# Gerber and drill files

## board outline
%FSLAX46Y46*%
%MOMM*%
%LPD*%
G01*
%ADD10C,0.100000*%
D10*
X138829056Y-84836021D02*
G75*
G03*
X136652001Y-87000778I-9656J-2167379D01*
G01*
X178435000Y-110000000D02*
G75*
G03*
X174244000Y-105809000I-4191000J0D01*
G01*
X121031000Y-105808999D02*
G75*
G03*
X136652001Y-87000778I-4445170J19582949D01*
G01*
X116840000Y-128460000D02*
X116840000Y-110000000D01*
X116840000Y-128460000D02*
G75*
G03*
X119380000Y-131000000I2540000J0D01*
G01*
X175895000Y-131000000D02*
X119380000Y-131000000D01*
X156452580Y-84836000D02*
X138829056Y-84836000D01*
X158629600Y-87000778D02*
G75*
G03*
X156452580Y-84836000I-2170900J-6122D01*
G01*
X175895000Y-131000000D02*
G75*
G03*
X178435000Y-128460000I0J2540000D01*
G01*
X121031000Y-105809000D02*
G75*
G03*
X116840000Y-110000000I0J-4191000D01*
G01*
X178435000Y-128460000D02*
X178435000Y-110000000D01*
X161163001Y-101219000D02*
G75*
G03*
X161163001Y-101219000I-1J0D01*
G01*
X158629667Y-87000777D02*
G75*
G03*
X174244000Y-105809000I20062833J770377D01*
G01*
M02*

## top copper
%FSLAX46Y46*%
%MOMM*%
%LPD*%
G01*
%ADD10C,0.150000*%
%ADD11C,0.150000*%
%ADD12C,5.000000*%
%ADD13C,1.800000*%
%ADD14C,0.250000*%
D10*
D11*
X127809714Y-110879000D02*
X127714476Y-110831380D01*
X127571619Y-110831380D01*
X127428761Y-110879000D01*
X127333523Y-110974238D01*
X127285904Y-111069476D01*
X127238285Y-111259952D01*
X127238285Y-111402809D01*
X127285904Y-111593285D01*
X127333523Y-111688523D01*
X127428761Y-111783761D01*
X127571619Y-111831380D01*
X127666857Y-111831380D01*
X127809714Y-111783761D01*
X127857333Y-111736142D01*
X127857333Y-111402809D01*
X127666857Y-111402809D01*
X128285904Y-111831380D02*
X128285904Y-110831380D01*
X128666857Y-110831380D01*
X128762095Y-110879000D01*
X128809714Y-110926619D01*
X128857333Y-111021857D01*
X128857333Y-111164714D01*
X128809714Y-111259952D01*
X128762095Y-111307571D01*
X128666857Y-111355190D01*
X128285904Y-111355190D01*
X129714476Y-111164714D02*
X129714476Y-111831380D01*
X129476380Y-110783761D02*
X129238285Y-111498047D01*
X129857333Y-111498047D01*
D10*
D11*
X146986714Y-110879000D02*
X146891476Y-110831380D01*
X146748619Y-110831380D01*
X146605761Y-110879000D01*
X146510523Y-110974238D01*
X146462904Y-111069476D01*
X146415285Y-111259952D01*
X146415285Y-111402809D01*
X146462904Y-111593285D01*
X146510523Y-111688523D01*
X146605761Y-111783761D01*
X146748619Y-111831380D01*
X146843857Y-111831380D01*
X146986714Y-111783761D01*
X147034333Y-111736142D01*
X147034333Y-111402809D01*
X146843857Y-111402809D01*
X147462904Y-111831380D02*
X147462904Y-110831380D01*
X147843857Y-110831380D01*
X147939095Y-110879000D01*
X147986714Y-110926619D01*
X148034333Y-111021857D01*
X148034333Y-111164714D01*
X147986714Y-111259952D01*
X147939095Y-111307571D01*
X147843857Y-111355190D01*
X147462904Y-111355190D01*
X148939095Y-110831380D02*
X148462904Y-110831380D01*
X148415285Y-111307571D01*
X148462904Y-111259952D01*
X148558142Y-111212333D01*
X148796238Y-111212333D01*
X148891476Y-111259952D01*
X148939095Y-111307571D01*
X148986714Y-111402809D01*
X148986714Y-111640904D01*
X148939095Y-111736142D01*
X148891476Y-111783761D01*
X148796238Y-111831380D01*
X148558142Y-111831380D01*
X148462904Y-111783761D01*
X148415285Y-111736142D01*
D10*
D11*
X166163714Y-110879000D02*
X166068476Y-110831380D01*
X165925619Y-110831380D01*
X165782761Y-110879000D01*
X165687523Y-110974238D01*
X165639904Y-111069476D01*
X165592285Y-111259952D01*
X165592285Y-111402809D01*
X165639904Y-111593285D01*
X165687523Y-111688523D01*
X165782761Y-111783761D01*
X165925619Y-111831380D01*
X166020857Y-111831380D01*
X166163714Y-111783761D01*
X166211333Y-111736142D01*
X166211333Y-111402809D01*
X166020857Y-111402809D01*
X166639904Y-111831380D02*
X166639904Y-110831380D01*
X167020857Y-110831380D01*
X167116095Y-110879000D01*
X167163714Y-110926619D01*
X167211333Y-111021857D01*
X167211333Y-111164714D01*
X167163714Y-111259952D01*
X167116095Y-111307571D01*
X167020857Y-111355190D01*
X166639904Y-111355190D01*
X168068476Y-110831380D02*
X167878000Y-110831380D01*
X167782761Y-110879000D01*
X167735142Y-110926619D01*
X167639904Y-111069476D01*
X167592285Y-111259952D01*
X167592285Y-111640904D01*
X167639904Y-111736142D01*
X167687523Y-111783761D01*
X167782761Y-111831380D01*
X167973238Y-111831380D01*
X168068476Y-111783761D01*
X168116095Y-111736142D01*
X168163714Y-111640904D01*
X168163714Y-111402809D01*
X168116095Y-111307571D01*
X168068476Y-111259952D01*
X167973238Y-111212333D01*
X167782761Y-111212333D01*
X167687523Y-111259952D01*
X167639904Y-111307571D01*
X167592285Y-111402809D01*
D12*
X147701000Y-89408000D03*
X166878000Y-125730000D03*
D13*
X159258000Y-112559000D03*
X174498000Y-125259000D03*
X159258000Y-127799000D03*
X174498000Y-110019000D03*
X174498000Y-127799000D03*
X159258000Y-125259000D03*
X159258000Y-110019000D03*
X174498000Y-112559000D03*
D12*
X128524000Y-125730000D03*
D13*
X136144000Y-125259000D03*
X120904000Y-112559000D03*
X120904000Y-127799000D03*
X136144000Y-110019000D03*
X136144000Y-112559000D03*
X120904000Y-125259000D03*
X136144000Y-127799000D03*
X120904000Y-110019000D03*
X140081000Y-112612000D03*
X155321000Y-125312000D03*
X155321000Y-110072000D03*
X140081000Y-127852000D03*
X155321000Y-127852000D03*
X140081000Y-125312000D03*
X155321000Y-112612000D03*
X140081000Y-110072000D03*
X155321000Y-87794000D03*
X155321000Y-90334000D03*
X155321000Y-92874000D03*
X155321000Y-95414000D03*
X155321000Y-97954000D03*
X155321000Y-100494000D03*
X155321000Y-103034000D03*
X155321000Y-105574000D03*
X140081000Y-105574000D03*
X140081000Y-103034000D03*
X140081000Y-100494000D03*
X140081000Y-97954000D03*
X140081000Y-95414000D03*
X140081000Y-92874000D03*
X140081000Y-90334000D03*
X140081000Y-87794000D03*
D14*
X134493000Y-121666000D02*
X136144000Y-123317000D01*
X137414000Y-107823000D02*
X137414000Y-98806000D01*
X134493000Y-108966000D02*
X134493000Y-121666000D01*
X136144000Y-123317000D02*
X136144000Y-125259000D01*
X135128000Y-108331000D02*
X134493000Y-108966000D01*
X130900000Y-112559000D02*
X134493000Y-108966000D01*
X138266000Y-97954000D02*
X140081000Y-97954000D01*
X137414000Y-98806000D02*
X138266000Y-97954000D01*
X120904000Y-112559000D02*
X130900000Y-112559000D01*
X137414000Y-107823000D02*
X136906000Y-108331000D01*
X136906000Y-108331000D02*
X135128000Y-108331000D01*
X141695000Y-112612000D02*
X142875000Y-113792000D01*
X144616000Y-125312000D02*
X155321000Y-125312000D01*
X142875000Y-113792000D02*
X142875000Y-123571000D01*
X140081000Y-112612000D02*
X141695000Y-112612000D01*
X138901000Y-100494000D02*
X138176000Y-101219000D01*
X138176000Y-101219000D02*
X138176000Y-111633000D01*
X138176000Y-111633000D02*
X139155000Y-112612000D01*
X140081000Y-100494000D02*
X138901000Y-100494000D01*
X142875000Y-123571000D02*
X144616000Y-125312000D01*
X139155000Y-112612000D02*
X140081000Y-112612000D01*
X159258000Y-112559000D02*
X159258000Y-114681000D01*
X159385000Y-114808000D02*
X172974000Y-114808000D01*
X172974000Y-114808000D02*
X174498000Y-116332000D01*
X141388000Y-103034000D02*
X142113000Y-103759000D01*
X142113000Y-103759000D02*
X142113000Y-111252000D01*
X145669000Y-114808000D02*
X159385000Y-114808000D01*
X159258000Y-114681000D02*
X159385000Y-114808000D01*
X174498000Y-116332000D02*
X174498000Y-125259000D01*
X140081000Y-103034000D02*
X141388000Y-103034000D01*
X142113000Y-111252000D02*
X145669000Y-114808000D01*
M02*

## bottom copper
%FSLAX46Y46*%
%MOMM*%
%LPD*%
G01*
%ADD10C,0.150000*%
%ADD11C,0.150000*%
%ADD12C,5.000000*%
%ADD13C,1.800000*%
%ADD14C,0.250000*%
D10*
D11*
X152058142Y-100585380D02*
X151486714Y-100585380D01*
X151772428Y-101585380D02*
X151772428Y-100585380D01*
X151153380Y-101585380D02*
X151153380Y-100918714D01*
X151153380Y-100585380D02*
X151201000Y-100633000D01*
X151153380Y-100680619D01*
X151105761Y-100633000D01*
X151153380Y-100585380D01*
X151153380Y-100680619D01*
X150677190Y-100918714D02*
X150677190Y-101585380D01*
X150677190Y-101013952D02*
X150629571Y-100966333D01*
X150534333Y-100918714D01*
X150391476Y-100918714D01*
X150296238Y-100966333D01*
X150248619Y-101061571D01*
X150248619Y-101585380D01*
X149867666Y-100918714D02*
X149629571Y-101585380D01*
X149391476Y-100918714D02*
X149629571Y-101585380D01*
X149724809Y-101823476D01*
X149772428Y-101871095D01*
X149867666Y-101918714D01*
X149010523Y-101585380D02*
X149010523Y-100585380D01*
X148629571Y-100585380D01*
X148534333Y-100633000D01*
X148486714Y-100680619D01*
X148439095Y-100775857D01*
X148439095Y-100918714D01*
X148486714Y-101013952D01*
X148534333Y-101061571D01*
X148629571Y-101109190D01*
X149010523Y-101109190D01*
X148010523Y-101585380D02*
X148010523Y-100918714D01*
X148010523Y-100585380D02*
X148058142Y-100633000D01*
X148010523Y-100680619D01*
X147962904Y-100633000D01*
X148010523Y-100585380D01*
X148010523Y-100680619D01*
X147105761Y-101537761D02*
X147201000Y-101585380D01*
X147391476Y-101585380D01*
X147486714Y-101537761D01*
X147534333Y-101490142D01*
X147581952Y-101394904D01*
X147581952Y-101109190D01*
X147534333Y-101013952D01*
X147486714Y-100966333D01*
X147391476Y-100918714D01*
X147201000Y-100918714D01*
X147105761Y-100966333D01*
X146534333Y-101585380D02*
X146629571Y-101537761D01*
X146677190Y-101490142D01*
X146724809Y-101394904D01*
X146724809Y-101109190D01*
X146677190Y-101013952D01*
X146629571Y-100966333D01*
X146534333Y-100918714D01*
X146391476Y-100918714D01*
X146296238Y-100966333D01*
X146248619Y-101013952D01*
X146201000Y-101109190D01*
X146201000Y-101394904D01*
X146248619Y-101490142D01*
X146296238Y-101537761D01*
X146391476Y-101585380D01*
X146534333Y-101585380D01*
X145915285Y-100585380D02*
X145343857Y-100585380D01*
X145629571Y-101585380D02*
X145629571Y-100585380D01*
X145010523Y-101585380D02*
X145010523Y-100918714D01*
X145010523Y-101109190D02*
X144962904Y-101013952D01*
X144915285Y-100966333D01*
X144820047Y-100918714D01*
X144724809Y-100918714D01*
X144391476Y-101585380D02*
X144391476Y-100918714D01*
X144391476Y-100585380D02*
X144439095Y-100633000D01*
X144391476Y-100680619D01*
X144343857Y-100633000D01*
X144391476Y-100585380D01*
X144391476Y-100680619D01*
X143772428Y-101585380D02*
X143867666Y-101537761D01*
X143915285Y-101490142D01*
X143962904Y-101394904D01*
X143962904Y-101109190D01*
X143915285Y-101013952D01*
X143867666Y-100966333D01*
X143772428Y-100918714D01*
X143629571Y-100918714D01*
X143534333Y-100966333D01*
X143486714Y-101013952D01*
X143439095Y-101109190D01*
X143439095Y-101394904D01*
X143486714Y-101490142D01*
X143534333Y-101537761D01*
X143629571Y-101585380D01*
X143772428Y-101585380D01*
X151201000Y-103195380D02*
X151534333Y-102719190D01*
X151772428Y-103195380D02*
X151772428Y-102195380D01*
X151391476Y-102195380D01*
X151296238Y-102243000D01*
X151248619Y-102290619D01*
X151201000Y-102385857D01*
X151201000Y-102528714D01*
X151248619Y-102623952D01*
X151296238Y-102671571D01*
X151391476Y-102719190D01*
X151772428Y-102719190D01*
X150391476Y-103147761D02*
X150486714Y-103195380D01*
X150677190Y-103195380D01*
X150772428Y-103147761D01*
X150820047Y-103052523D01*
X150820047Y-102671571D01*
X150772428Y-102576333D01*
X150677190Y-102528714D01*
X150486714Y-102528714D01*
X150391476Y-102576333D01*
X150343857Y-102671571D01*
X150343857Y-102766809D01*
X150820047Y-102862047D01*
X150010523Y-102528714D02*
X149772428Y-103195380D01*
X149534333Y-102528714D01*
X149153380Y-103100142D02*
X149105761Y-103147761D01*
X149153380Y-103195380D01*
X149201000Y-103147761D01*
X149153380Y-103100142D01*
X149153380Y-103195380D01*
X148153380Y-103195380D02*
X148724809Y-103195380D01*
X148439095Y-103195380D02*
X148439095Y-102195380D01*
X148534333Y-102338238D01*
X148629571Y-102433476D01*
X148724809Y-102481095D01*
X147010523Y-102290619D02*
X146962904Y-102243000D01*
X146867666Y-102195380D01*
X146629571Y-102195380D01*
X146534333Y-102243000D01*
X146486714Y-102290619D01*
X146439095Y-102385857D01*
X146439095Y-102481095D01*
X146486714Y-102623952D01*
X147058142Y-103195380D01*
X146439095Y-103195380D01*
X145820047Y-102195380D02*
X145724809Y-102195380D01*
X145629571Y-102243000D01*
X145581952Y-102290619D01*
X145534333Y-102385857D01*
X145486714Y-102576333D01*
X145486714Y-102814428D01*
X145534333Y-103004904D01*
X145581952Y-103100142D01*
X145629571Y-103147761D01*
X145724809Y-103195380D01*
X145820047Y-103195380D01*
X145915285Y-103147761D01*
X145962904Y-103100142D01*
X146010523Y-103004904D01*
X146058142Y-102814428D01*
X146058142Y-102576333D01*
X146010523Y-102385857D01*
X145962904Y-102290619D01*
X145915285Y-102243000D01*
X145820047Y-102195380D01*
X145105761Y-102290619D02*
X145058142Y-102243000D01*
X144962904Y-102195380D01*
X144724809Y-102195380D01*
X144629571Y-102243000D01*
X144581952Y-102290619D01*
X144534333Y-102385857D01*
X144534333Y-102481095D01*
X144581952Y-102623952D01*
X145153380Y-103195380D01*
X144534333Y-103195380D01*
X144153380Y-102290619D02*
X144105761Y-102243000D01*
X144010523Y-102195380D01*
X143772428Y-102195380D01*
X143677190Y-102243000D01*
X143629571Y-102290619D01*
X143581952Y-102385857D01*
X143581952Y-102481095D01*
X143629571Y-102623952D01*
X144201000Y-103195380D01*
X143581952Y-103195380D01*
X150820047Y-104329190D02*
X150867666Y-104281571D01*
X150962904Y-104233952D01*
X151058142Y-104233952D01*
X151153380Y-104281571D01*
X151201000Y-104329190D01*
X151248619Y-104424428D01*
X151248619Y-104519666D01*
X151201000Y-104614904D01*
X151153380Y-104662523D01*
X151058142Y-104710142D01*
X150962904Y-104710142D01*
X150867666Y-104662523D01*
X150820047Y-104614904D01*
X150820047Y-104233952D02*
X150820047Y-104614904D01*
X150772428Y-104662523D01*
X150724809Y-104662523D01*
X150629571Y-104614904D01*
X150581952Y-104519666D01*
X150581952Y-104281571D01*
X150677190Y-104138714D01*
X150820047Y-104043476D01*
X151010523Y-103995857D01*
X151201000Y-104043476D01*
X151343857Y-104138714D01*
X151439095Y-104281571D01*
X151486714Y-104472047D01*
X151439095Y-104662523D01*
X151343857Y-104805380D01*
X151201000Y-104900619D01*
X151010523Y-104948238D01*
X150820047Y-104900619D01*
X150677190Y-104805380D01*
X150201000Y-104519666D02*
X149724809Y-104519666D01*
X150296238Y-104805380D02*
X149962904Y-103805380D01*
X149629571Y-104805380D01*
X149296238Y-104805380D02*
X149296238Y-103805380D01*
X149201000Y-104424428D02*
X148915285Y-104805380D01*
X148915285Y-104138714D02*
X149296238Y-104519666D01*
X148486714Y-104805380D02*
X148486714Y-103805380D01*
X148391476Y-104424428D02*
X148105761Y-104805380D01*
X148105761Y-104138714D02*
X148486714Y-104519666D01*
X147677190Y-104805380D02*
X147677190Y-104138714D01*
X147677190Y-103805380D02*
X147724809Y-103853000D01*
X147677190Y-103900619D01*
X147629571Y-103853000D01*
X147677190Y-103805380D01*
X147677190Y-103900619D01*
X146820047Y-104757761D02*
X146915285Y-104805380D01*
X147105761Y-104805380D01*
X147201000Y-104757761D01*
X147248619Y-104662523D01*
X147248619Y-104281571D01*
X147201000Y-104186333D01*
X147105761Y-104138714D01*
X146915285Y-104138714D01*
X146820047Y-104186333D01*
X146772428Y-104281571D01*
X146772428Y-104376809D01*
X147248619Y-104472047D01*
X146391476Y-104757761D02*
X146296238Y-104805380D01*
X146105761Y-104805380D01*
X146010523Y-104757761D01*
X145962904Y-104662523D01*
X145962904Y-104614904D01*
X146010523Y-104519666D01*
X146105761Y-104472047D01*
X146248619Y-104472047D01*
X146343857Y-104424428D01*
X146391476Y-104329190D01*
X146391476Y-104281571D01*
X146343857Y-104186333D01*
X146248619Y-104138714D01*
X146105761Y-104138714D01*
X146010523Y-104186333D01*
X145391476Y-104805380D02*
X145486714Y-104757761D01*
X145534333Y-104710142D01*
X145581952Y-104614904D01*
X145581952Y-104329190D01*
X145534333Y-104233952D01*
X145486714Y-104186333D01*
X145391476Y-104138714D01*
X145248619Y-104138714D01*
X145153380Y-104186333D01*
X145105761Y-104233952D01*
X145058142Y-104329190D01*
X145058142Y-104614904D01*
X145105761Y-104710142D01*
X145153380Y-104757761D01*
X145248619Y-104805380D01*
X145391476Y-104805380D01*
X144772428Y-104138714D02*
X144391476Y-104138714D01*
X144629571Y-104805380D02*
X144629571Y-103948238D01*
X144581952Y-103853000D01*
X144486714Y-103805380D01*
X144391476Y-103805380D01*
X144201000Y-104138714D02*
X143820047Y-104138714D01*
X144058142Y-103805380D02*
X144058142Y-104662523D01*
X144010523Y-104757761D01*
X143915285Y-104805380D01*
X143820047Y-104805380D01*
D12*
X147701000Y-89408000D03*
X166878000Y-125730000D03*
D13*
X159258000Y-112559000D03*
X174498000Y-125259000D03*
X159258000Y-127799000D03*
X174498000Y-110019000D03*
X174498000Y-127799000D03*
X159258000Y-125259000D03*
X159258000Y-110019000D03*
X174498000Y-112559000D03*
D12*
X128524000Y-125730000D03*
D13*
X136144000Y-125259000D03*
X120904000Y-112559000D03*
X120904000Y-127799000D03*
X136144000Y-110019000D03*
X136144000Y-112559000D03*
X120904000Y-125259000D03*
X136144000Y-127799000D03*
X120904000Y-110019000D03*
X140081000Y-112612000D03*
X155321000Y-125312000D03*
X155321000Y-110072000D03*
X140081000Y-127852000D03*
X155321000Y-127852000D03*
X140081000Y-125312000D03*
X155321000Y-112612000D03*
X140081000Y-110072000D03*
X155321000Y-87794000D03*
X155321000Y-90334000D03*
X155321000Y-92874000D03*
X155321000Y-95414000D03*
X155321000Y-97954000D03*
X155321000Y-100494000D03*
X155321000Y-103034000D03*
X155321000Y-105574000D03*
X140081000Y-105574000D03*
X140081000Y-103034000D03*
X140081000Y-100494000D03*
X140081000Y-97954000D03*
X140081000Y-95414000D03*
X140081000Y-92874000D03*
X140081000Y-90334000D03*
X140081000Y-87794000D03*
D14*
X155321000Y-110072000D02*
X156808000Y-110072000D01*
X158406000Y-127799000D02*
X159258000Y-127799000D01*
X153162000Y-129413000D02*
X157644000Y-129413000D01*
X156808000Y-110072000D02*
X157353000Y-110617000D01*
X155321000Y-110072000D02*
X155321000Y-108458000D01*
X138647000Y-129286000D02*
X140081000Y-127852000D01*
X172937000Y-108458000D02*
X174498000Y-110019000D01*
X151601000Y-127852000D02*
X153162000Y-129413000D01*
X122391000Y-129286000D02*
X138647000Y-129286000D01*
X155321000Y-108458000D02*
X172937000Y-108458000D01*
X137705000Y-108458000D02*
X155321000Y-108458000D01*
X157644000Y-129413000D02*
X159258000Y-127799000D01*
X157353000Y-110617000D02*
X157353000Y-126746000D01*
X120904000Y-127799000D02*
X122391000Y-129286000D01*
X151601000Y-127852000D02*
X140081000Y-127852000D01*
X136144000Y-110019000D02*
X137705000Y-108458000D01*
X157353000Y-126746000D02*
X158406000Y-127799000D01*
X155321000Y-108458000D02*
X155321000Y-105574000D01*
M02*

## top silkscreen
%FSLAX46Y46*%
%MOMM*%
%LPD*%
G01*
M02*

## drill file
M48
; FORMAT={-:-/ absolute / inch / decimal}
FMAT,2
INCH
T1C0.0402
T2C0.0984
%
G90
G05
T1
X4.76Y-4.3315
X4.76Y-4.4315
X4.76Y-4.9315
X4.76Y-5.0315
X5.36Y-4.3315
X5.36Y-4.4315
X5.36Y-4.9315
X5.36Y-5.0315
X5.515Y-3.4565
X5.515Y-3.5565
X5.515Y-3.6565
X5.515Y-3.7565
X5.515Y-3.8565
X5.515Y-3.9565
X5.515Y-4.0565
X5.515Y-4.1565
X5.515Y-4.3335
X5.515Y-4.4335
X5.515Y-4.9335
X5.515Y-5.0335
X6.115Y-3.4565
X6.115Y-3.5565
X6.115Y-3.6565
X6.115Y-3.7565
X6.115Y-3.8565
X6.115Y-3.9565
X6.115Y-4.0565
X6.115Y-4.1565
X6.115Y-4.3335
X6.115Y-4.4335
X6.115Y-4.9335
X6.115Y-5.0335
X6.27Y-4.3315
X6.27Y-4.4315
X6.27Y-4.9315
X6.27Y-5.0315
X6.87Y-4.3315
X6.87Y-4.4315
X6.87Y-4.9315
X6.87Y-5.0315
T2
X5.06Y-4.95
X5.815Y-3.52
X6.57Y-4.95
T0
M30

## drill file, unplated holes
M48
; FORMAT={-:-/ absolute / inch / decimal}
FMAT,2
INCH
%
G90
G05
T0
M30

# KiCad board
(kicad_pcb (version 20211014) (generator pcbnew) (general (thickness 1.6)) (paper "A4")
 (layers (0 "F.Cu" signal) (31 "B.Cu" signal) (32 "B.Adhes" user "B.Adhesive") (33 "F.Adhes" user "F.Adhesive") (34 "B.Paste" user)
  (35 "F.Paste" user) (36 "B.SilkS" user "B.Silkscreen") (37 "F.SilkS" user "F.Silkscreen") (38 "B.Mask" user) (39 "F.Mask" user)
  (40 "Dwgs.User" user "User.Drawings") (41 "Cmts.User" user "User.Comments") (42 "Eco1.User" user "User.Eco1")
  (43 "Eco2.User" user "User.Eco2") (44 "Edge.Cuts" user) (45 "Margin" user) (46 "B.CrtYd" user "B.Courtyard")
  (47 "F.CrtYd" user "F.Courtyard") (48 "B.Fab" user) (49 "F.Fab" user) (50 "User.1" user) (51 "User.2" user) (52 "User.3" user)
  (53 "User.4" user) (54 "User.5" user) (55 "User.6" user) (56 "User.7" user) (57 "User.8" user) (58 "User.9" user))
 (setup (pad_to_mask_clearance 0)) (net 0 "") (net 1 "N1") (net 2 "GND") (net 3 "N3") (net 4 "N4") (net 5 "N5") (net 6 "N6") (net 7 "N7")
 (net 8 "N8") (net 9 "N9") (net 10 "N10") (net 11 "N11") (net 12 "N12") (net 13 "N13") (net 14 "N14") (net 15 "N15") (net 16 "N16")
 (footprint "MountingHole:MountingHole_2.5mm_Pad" (layer "F.Cu") (at 147.701 89.408)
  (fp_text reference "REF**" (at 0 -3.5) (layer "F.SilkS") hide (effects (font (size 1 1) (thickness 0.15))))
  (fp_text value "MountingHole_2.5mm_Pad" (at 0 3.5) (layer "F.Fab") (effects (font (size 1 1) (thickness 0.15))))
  (pad "1" thru_hole circle (at 0 0) (size 5 5) (drill 2.5) (layers *.Cu *.Mask)))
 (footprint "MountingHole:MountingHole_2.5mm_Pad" (layer "F.Cu") (at 166.878 125.73)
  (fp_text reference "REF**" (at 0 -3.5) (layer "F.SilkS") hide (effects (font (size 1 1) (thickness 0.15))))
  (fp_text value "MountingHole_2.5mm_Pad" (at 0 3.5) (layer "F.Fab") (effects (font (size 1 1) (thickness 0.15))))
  (pad "1" thru_hole circle (at 0 0) (size 5 5) (drill 2.5) (layers *.Cu *.Mask)))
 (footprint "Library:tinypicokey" (layer "F.Cu") (at 166.878 104.939)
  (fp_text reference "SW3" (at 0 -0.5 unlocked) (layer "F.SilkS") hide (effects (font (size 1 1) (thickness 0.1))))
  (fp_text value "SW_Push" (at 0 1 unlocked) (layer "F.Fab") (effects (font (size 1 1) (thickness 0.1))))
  (pad "1" thru_hole circle (at -7.62 7.62) (size 1.8 1.8) (drill 1.02) (layers *.Cu *.Mask) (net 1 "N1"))
  (pad "1" thru_hole circle (at 7.62 20.32) (size 1.8 1.8) (drill 1.02) (layers *.Cu *.Mask) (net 1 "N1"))
  (pad "2" thru_hole circle (at -7.62 22.86) (size 1.8 1.8) (drill 1.02) (layers *.Cu *.Mask) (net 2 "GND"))
  (pad "2" thru_hole circle (at 7.62 5.08) (size 1.8 1.8) (drill 1.02) (layers *.Cu *.Mask) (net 2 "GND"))
  (pad "3" thru_hole circle (at 7.62 22.86) (size 1.8 1.8) (drill 1.02) (layers *.Cu *.Mask))
  (pad "3" thru_hole circle (at -7.62 20.32) (size 1.8 1.8) (drill 1.02) (layers *.Cu *.Mask))
  (pad "3" thru_hole circle (at -7.62 5.08) (size 1.8 1.8) (drill 1.02) (layers *.Cu *.Mask))
  (pad "3" thru_hole circle (at 7.62 7.62) (size 1.8 1.8) (drill 1.02) (layers *.Cu *.Mask)))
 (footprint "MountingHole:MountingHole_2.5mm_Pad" (layer "F.Cu") (at 128.524 125.73)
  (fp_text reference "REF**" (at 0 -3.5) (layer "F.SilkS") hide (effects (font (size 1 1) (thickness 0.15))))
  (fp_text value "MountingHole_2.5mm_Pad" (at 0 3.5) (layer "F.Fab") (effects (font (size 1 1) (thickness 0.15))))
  (pad "1" thru_hole circle (at 0 0) (size 5 5) (drill 2.5) (layers *.Cu *.Mask)))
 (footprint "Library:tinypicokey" (layer "F.Cu") (at 128.524 104.939)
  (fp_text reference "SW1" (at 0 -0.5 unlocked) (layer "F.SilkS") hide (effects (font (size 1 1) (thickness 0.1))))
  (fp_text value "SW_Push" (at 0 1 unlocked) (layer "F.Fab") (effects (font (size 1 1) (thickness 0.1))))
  (pad "1" thru_hole circle (at 7.62 20.32) (size 1.8 1.8) (drill 1.02) (layers *.Cu *.Mask) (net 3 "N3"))
  (pad "1" thru_hole circle (at -7.62 7.62) (size 1.8 1.8) (drill 1.02) (layers *.Cu *.Mask) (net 3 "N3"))
  (pad "2" thru_hole circle (at -7.62 22.86) (size 1.8 1.8) (drill 1.02) (layers *.Cu *.Mask) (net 2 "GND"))
  (pad "2" thru_hole circle (at 7.62 5.08) (size 1.8 1.8) (drill 1.02) (layers *.Cu *.Mask) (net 2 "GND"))
  (pad "3" thru_hole circle (at 7.62 7.62) (size 1.8 1.8) (drill 1.02) (layers *.Cu *.Mask))
  (pad "3" thru_hole circle (at -7.62 20.32) (size 1.8 1.8) (drill 1.02) (layers *.Cu *.Mask))
  (pad "3" thru_hole circle (at 7.62 22.86) (size 1.8 1.8) (drill 1.02) (layers *.Cu *.Mask))
  (pad "3" thru_hole circle (at -7.62 5.08) (size 1.8 1.8) (drill 1.02) (layers *.Cu *.Mask)))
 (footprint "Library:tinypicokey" (layer "F.Cu") (at 147.701 132.932 180)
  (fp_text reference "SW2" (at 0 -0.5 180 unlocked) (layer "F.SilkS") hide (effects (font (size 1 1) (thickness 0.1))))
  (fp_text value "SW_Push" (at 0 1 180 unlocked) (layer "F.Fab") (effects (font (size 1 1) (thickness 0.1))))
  (pad "1" thru_hole circle (at 7.62 20.32 180) (size 1.8 1.8) (drill 1.02) (layers *.Cu *.Mask) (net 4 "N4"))
  (pad "1" thru_hole circle (at -7.62 7.62 180) (size 1.8 1.8) (drill 1.02) (layers *.Cu *.Mask) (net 4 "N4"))
  (pad "2" thru_hole circle (at -7.62 22.86 180) (size 1.8 1.8) (drill 1.02) (layers *.Cu *.Mask) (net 2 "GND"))
  (pad "2" thru_hole circle (at 7.62 5.08 180) (size 1.8 1.8) (drill 1.02) (layers *.Cu *.Mask) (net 2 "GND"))
  (pad "3" thru_hole circle (at -7.62 5.08 180) (size 1.8 1.8) (drill 1.02) (layers *.Cu *.Mask))
  (pad "3" thru_hole circle (at 7.62 7.62 180) (size 1.8 1.8) (drill 1.02) (layers *.Cu *.Mask))
  (pad "3" thru_hole circle (at -7.62 20.32 180) (size 1.8 1.8) (drill 1.02) (layers *.Cu *.Mask))
  (pad "3" thru_hole circle (at 7.62 22.86 180) (size 1.8 1.8) (drill 1.02) (layers *.Cu *.Mask)))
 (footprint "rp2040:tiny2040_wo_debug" (layer "B.Cu") (at 147.701 82.714 180)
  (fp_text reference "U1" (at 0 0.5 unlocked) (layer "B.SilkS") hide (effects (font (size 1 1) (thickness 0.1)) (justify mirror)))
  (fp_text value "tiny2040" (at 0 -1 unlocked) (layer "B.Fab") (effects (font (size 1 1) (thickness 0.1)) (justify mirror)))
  (pad "1" thru_hole circle locked (at -7.62 -5.08 180) (size 1.8 1.8) (drill 1.02) (layers *.Cu *.Mask) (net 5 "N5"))
  (pad "2" thru_hole circle locked (at -7.62 -7.62 180) (size 1.8 1.8) (drill 1.02) (layers *.Cu *.Mask) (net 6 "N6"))
  (pad "3" thru_hole circle locked (at -7.62 -10.16 180) (size 1.8 1.8) (drill 1.02) (layers *.Cu *.Mask) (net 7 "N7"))
  (pad "4" thru_hole circle locked (at -7.62 -12.7 180) (size 1.8 1.8) (drill 1.02) (layers *.Cu *.Mask) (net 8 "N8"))
  (pad "5" thru_hole circle locked (at -7.62 -15.24 180) (size 1.8 1.8) (drill 1.02) (layers *.Cu *.Mask) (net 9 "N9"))
  (pad "6" thru_hole circle locked (at -7.62 -17.78 180) (size 1.8 1.8) (drill 1.02) (layers *.Cu *.Mask) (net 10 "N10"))
  (pad "7" thru_hole circle locked (at -7.62 -20.32 180) (size 1.8 1.8) (drill 1.02) (layers *.Cu *.Mask) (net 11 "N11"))
  (pad "8" thru_hole circle locked (at -7.62 -22.86 180) (size 1.8 1.8) (drill 1.02) (layers *.Cu *.Mask) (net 2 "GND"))
  (pad "9" thru_hole circle locked (at 7.62 -22.86 180) (size 1.8 1.8) (drill 1.02) (layers *.Cu *.Mask) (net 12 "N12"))
  (pad "10" thru_hole circle locked (at 7.62 -20.32 180) (size 1.8 1.8) (drill 1.02) (layers *.Cu *.Mask) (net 1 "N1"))
  (pad "11" thru_hole circle locked (at 7.62 -17.78 180) (size 1.8 1.8) (drill 1.02) (layers *.Cu *.Mask) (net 4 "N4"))
  (pad "12" thru_hole circle locked (at 7.62 -15.24 180) (size 1.8 1.8) (drill 1.02) (layers *.Cu *.Mask) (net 3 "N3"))
  (pad "13" thru_hole circle locked (at 7.62 -12.7 180) (size 1.8 1.8) (drill 1.02) (layers *.Cu *.Mask) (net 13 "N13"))
  (pad "14" thru_hole circle locked (at 7.62 -10.16 180) (size 1.8 1.8) (drill 1.02) (layers *.Cu *.Mask) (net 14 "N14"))
  (pad "15" thru_hole circle locked (at 7.62 -7.62 180) (size 1.8 1.8) (drill 1.02) (layers *.Cu *.Mask) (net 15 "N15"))
  (pad "16" thru_hole circle locked (at 7.62 -5.08 180) (size 1.8 1.8) (drill 1.02) (layers *.Cu *.Mask) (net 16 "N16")))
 (gr_arc (start 136.652001 87.000778) (mid 137.291161 85.466473) (end 138.829056 84.836) (layer "Edge.Cuts") (width 0.1))
 (gr_arc (start 174.244 105.809) (mid 177.207485 107.036515) (end 178.435 110) (layer "Edge.Cuts") (width 0.1))
 (gr_arc (start 136.652001 87.000778) (mid 132.033766 99.056197) (end 121.031 105.809) (layer "Edge.Cuts") (width 0.1))
 (gr_line (start 116.84 128.46) (end 116.84 110) (layer "Edge.Cuts") (width 0.1))
 (gr_arc (start 119.38 131) (mid 117.583949 130.256051) (end 116.84 128.46) (layer "Edge.Cuts") (width 0.1))
 (gr_line (start 175.895 131) (end 119.38 131) (layer "Edge.Cuts") (width 0.1))
 (gr_line (start 156.45258 84.836) (end 138.829056 84.836) (layer "Edge.Cuts") (width 0.1))
 (gr_arc (start 156.45258 84.836) (mid 157.989448 85.467506) (end 158.629635 87.000778) (layer "Edge.Cuts") (width 0.1))
 (gr_arc (start 178.435 128.46) (mid 177.691051 130.256051) (end 175.895 131) (layer "Edge.Cuts") (width 0.1))
 (gr_arc (start 116.84 110) (mid 118.067515 107.036515) (end 121.031 105.809) (layer "Edge.Cuts") (width 0.1))
 (gr_line (start 178.435 128.46) (end 178.435 110) (layer "Edge.Cuts") (width 0.1))
 (gr_circle (center 161.163 101.219) (end 161.163 101.219) (layer "Edge.Cuts") (width 0.1) (fill none))
 (gr_arc (start 174.244 105.809) (mid 163.244552 99.05507) (end 158.629635 87.000778) (layer "Edge.Cuts") (width 0.1))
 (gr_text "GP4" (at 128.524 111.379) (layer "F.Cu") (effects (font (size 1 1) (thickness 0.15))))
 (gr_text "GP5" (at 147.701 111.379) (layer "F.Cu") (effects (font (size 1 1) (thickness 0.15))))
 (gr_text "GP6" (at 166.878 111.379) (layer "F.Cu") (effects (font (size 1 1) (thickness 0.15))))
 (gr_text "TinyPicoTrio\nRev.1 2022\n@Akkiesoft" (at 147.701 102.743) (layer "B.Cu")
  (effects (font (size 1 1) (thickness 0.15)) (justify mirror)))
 (segment (start 155.321 110.072) (end 156.808 110.072) (width 0.25) (layer "B.Cu") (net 2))
 (segment (start 158.406 127.799) (end 159.258 127.799) (width 0.25) (layer "B.Cu") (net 2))
 (segment (start 153.162 129.413) (end 157.644 129.413) (width 0.25) (layer "B.Cu") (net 2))
 (segment (start 156.808 110.072) (end 157.353 110.617) (width 0.25) (layer "B.Cu") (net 2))
 (segment (start 155.321 110.072) (end 155.321 108.458) (width 0.25) (layer "B.Cu") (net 2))
 (segment (start 138.647 129.286) (end 140.081 127.852) (width 0.25) (layer "B.Cu") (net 2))
 (segment (start 172.937 108.458) (end 174.498 110.019) (width 0.25) (layer "B.Cu") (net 2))
 (segment (start 151.601 127.852) (end 153.162 129.413) (width 0.25) (layer "B.Cu") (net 2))
 (segment (start 122.391 129.286) (end 138.647 129.286) (width 0.25) (layer "B.Cu") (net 2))
 (segment (start 155.321 108.458) (end 172.937 108.458) (width 0.25) (layer "B.Cu") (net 2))
 (segment (start 137.705 108.458) (end 155.321 108.458) (width 0.25) (layer "B.Cu") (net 2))
 (segment (start 157.644 129.413) (end 159.258 127.799) (width 0.25) (layer "B.Cu") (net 2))
 (segment (start 157.353 110.617) (end 157.353 126.746) (width 0.25) (layer "B.Cu") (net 2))
 (segment (start 120.904 127.799) (end 122.391 129.286) (width 0.25) (layer "B.Cu") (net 2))
 (segment (start 151.601 127.852) (end 140.081 127.852) (width 0.25) (layer "B.Cu") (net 2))
 (segment (start 136.144 110.019) (end 137.705 108.458) (width 0.25) (layer "B.Cu") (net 2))
 (segment (start 157.353 126.746) (end 158.406 127.799) (width 0.25) (layer "B.Cu") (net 2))
 (segment (start 155.321 108.458) (end 155.321 105.574) (width 0.25) (layer "B.Cu") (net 2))
 (segment (start 134.493 121.666) (end 136.144 123.317) (width 0.25) (layer "F.Cu") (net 3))
 (segment (start 137.414 107.823) (end 137.414 98.806) (width 0.25) (layer "F.Cu") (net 3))
 (segment (start 134.493 108.966) (end 134.493 121.666) (width 0.25) (layer "F.Cu") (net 3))
 (segment (start 136.144 123.317) (end 136.144 125.259) (width 0.25) (layer "F.Cu") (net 3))
 (segment (start 135.128 108.331) (end 134.493 108.966) (width 0.25) (layer "F.Cu") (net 3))
 (segment (start 130.9 112.559) (end 134.493 108.966) (width 0.25) (layer "F.Cu") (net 3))
 (segment (start 138.266 97.954) (end 140.081 97.954) (width 0.25) (layer "F.Cu") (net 3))
 (segment (start 137.414 98.806) (end 138.266 97.954) (width 0.25) (layer "F.Cu") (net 3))
 (segment (start 120.904 112.559) (end 130.9 112.559) (width 0.25) (layer "F.Cu") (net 3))
 (segment (start 137.414 107.823) (end 136.906 108.331) (width 0.25) (layer "F.Cu") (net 3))
 (segment (start 136.906 108.331) (end 135.128 108.331) (width 0.25) (layer "F.Cu") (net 3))
 (segment (start 141.695 112.612) (end 142.875 113.792) (width 0.25) (layer "F.Cu") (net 4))
 (segment (start 144.616 125.312) (end 155.321 125.312) (width 0.25) (layer "F.Cu") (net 4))
 (segment (start 142.875 113.792) (end 142.875 123.571) (width 0.25) (layer "F.Cu") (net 4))
 (segment (start 140.081 112.612) (end 141.695 112.612) (width 0.25) (layer "F.Cu") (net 4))
 (segment (start 138.901 100.494) (end 138.176 101.219) (width 0.25) (layer "F.Cu") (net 4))
 (segment (start 138.176 101.219) (end 138.176 111.633) (width 0.25) (layer "F.Cu") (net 4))
 (segment (start 138.176 111.633) (end 139.155 112.612) (width 0.25) (layer "F.Cu") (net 4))
 (segment (start 140.081 100.494) (end 138.901 100.494) (width 0.25) (layer "F.Cu") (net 4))
 (segment (start 142.875 123.571) (end 144.616 125.312) (width 0.25) (layer "F.Cu") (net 4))
 (segment (start 139.155 112.612) (end 140.081 112.612) (width 0.25) (layer "F.Cu") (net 4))
 (segment (start 159.258 112.559) (end 159.258 114.681) (width 0.25) (layer "F.Cu") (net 1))
 (segment (start 159.385 114.808) (end 172.974 114.808) (width 0.25) (layer "F.Cu") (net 1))
 (segment (start 172.974 114.808) (end 174.498 116.332) (width 0.25) (layer "F.Cu") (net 1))
 (segment (start 141.388 103.034) (end 142.113 103.759) (width 0.25) (layer "F.Cu") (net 1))
 (segment (start 142.113 103.759) (end 142.113 111.252) (width 0.25) (layer "F.Cu") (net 1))
 (segment (start 145.669 114.808) (end 159.385 114.808) (width 0.25) (layer "F.Cu") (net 1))
 (segment (start 159.258 114.681) (end 159.385 114.808) (width 0.25) (layer "F.Cu") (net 1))
 (segment (start 174.498 116.332) (end 174.498 125.259) (width 0.25) (layer "F.Cu") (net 1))
 (segment (start 140.081 103.034) (end 141.388 103.034) (width 0.25) (layer "F.Cu") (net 1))
 (segment (start 142.113 111.252) (end 145.669 114.808) (width 0.25) (layer "F.Cu") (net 1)))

